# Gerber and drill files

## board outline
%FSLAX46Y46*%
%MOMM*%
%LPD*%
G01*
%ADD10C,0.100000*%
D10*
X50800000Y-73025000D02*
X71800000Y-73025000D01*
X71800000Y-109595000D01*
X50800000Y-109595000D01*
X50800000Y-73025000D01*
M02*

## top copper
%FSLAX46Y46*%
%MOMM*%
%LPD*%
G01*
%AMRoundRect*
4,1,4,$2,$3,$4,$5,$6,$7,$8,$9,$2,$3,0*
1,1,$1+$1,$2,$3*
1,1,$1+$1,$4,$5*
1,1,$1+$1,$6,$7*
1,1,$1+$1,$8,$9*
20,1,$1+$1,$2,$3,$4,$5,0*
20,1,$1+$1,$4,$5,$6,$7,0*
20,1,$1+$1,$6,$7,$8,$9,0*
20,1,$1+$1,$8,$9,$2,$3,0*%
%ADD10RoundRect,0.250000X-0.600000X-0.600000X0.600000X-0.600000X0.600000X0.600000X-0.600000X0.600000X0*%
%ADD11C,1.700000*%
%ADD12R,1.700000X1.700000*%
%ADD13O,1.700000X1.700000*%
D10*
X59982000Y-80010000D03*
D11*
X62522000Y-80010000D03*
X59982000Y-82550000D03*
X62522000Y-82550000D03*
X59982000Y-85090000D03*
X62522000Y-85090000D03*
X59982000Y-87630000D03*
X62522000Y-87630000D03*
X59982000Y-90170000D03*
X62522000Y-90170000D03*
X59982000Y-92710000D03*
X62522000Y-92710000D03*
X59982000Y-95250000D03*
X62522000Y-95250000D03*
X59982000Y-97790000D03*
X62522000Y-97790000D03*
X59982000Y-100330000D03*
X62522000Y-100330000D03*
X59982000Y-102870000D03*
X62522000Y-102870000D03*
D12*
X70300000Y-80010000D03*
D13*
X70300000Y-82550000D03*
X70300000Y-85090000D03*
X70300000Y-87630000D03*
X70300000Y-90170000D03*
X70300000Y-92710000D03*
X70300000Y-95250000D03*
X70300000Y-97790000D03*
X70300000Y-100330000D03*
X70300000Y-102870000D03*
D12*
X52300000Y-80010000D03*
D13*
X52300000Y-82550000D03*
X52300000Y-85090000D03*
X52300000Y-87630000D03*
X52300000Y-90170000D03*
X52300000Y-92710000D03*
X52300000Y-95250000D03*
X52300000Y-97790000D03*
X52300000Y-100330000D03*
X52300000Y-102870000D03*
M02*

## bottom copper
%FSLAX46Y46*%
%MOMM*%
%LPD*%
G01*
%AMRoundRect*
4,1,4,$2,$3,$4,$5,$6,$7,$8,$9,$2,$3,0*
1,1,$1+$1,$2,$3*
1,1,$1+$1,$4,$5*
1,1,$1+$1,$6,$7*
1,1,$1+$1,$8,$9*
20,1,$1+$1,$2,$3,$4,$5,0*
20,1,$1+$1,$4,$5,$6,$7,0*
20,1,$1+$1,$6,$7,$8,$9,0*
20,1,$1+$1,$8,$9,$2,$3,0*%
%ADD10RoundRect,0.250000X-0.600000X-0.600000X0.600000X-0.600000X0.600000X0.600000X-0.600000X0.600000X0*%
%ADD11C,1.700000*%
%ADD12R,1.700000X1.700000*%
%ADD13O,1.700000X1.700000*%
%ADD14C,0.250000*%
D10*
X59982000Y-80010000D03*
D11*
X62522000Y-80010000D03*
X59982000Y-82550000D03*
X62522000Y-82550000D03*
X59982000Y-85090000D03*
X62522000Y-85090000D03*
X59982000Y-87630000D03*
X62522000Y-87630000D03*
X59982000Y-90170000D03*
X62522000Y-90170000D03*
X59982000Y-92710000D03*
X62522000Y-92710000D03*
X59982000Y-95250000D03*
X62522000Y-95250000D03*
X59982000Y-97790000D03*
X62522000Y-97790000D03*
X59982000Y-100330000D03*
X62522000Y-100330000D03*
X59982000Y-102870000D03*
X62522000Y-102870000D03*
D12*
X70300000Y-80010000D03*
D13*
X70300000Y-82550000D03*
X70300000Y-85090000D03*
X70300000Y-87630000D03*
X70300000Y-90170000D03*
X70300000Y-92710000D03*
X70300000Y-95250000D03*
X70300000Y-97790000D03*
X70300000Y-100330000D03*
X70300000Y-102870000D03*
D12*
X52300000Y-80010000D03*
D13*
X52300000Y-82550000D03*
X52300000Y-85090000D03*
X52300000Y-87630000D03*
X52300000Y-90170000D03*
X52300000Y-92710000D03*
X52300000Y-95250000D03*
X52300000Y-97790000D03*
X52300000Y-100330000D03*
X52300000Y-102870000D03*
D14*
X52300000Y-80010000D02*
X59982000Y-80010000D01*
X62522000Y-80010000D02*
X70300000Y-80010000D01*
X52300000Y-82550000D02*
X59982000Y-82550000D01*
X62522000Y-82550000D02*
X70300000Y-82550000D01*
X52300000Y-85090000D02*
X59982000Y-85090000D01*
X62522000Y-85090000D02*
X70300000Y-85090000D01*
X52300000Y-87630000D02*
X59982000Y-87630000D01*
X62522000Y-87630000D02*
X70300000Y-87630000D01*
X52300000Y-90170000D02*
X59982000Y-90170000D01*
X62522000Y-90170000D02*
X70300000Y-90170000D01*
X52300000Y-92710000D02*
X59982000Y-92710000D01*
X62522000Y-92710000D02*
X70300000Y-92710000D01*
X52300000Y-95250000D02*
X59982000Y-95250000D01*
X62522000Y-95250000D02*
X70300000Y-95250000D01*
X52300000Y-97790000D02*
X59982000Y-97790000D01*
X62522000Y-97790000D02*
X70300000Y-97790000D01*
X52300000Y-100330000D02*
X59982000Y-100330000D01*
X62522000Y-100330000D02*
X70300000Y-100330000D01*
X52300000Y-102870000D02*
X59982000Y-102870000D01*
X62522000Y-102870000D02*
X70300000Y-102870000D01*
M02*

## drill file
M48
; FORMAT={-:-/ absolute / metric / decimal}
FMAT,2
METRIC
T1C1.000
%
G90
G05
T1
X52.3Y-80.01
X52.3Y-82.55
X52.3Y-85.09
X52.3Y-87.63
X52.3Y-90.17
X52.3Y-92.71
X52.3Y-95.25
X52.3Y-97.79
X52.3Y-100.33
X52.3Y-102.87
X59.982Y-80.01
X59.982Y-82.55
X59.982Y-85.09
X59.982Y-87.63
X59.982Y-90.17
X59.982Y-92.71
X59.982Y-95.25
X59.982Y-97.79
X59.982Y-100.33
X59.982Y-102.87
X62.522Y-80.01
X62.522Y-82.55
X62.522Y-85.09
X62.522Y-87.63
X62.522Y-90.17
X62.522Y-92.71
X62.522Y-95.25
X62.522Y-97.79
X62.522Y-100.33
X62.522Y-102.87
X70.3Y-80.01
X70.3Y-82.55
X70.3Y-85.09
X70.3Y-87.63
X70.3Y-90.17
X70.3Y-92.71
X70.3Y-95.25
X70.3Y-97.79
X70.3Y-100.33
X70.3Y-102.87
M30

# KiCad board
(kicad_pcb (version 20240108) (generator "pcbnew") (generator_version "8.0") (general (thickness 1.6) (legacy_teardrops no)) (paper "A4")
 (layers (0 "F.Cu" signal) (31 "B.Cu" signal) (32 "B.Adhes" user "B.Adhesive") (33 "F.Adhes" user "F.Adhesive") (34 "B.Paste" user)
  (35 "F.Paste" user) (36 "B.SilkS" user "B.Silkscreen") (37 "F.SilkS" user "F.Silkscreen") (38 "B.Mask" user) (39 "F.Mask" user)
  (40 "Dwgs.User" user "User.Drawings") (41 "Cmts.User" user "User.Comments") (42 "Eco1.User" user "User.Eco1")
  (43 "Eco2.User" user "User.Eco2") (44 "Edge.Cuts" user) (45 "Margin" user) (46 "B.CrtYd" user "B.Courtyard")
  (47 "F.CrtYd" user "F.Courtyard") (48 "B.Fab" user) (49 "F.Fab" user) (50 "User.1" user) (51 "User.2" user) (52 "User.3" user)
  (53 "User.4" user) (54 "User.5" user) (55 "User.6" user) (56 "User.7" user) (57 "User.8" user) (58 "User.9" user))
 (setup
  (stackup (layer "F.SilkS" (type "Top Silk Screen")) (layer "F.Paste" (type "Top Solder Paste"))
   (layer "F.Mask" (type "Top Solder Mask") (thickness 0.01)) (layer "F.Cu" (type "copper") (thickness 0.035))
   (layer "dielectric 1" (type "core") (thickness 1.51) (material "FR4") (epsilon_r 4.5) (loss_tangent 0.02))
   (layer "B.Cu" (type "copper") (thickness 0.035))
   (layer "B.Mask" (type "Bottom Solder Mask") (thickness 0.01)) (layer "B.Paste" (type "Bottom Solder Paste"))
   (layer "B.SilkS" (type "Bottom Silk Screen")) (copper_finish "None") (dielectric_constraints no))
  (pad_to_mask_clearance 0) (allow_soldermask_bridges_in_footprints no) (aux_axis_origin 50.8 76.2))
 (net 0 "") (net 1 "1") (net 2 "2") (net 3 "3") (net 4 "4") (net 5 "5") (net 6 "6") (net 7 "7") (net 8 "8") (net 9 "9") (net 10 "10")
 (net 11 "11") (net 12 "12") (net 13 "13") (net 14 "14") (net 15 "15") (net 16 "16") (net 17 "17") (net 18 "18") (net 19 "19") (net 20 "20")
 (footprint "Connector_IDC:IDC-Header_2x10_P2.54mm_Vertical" (layer "F.Cu") (at 59.982 80.01)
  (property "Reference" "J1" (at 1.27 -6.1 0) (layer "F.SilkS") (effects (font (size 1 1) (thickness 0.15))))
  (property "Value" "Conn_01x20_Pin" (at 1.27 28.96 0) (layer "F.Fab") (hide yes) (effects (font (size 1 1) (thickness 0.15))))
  (pad "1" thru_hole roundrect (at 0 0) (size 1.7 1.7) (drill 1) (layers "*.Cu" "*.Mask") (remove_unused_layers no)
   (roundrect_rratio 0.147059) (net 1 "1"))
  (pad "2" thru_hole circle (at 2.54 0) (size 1.7 1.7) (drill 1) (layers "*.Cu" "*.Mask") (remove_unused_layers no) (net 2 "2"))
  (pad "3" thru_hole circle (at 0 2.54) (size 1.7 1.7) (drill 1) (layers "*.Cu" "*.Mask") (remove_unused_layers no) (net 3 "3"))
  (pad "4" thru_hole circle (at 2.54 2.54) (size 1.7 1.7) (drill 1) (layers "*.Cu" "*.Mask") (remove_unused_layers no) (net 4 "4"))
  (pad "5" thru_hole circle (at 0 5.08) (size 1.7 1.7) (drill 1) (layers "*.Cu" "*.Mask") (remove_unused_layers no) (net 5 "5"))
  (pad "6" thru_hole circle (at 2.54 5.08) (size 1.7 1.7) (drill 1) (layers "*.Cu" "*.Mask") (remove_unused_layers no) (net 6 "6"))
  (pad "7" thru_hole circle (at 0 7.62) (size 1.7 1.7) (drill 1) (layers "*.Cu" "*.Mask") (remove_unused_layers no) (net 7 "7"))
  (pad "8" thru_hole circle (at 2.54 7.62) (size 1.7 1.7) (drill 1) (layers "*.Cu" "*.Mask") (remove_unused_layers no) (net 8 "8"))
  (pad "9" thru_hole circle (at 0 10.16) (size 1.7 1.7) (drill 1) (layers "*.Cu" "*.Mask") (remove_unused_layers no) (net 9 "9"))
  (pad "10" thru_hole circle (at 2.54 10.16) (size 1.7 1.7) (drill 1) (layers "*.Cu" "*.Mask") (remove_unused_layers no) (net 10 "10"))
  (pad "11" thru_hole circle (at 0 12.7) (size 1.7 1.7) (drill 1) (layers "*.Cu" "*.Mask") (remove_unused_layers no) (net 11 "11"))
  (pad "12" thru_hole circle (at 2.54 12.7) (size 1.7 1.7) (drill 1) (layers "*.Cu" "*.Mask") (remove_unused_layers no) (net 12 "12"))
  (pad "13" thru_hole circle (at 0 15.24) (size 1.7 1.7) (drill 1) (layers "*.Cu" "*.Mask") (remove_unused_layers no) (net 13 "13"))
  (pad "14" thru_hole circle (at 2.54 15.24) (size 1.7 1.7) (drill 1) (layers "*.Cu" "*.Mask") (remove_unused_layers no) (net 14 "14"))
  (pad "15" thru_hole circle (at 0 17.78) (size 1.7 1.7) (drill 1) (layers "*.Cu" "*.Mask") (remove_unused_layers no) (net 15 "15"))
  (pad "16" thru_hole circle (at 2.54 17.78) (size 1.7 1.7) (drill 1) (layers "*.Cu" "*.Mask") (remove_unused_layers no) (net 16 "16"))
  (pad "17" thru_hole circle (at 0 20.32) (size 1.7 1.7) (drill 1) (layers "*.Cu" "*.Mask") (remove_unused_layers no) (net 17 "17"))
  (pad "18" thru_hole circle (at 2.54 20.32) (size 1.7 1.7) (drill 1) (layers "*.Cu" "*.Mask") (remove_unused_layers no) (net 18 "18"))
  (pad "19" thru_hole circle (at 0 22.86) (size 1.7 1.7) (drill 1) (layers "*.Cu" "*.Mask") (remove_unused_layers no) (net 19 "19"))
  (pad "20" thru_hole circle (at 2.54 22.86) (size 1.7 1.7) (drill 1) (layers "*.Cu" "*.Mask") (remove_unused_layers no) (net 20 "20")))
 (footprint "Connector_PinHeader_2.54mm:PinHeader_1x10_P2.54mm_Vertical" (layer "B.Cu") (at 70.3 80.01 180)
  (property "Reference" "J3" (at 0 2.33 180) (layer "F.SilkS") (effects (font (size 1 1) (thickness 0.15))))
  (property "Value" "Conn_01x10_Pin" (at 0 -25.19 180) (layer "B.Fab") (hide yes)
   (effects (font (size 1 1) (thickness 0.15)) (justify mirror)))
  (pad "1" thru_hole rect (at 0 0 180) (size 1.7 1.7) (drill 1) (layers "*.Cu" "*.Mask") (remove_unused_layers no) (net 2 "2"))
  (pad "2" thru_hole oval (at 0 -2.54 180) (size 1.7 1.7) (drill 1) (layers "*.Cu" "*.Mask") (remove_unused_layers no) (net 4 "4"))
  (pad "3" thru_hole oval (at 0 -5.08 180) (size 1.7 1.7) (drill 1) (layers "*.Cu" "*.Mask") (remove_unused_layers no) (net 6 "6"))
  (pad "4" thru_hole oval (at 0 -7.62 180) (size 1.7 1.7) (drill 1) (layers "*.Cu" "*.Mask") (remove_unused_layers no) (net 8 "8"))
  (pad "5" thru_hole oval (at 0 -10.16 180) (size 1.7 1.7) (drill 1) (layers "*.Cu" "*.Mask") (remove_unused_layers no) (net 10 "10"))
  (pad "6" thru_hole oval (at 0 -12.7 180) (size 1.7 1.7) (drill 1) (layers "*.Cu" "*.Mask") (remove_unused_layers no) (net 12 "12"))
  (pad "7" thru_hole oval (at 0 -15.24 180) (size 1.7 1.7) (drill 1) (layers "*.Cu" "*.Mask") (remove_unused_layers no) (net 14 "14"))
  (pad "8" thru_hole oval (at 0 -17.78 180) (size 1.7 1.7) (drill 1) (layers "*.Cu" "*.Mask") (remove_unused_layers no) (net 16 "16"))
  (pad "9" thru_hole oval (at 0 -20.32 180) (size 1.7 1.7) (drill 1) (layers "*.Cu" "*.Mask") (remove_unused_layers no) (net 18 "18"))
  (pad "10" thru_hole oval (at 0 -22.86 180) (size 1.7 1.7) (drill 1) (layers "*.Cu" "*.Mask") (remove_unused_layers no) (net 20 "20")))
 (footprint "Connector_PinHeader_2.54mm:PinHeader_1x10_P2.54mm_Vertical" (layer "B.Cu") (at 52.3 80.01 180)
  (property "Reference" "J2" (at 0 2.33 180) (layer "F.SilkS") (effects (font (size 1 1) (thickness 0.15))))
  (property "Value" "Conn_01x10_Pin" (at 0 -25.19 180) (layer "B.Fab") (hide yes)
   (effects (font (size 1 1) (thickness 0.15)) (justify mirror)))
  (pad "1" thru_hole rect (at 0 0 180) (size 1.7 1.7) (drill 1) (layers "*.Cu" "*.Mask") (remove_unused_layers no) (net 1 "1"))
  (pad "2" thru_hole oval (at 0 -2.54 180) (size 1.7 1.7) (drill 1) (layers "*.Cu" "*.Mask") (remove_unused_layers no) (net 3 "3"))
  (pad "3" thru_hole oval (at 0 -5.08 180) (size 1.7 1.7) (drill 1) (layers "*.Cu" "*.Mask") (remove_unused_layers no) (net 5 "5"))
  (pad "4" thru_hole oval (at 0 -7.62 180) (size 1.7 1.7) (drill 1) (layers "*.Cu" "*.Mask") (remove_unused_layers no) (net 7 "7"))
  (pad "5" thru_hole oval (at 0 -10.16 180) (size 1.7 1.7) (drill 1) (layers "*.Cu" "*.Mask") (remove_unused_layers no) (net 9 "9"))
  (pad "6" thru_hole oval (at 0 -12.7 180) (size 1.7 1.7) (drill 1) (layers "*.Cu" "*.Mask") (remove_unused_layers no) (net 11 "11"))
  (pad "7" thru_hole oval (at 0 -15.24 180) (size 1.7 1.7) (drill 1) (layers "*.Cu" "*.Mask") (remove_unused_layers no) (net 13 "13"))
  (pad "8" thru_hole oval (at 0 -17.78 180) (size 1.7 1.7) (drill 1) (layers "*.Cu" "*.Mask") (remove_unused_layers no) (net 15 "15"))
  (pad "9" thru_hole oval (at 0 -20.32 180) (size 1.7 1.7) (drill 1) (layers "*.Cu" "*.Mask") (remove_unused_layers no) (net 17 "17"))
  (pad "10" thru_hole oval (at 0 -22.86 180) (size 1.7 1.7) (drill 1) (layers "*.Cu" "*.Mask") (remove_unused_layers no) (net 19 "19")))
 (gr_rect (start 50.8 73.025) (end 71.8 109.595) (stroke (width 0.1) (type default)) (fill none) (layer "Edge.Cuts"))
 (segment (start 52.3 80.01) (end 59.982 80.01) (width 0.25) (layer "B.Cu") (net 1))
 (segment (start 62.522 80.01) (end 70.3 80.01) (width 0.25) (layer "B.Cu") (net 2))
 (segment (start 52.3 82.55) (end 59.982 82.55) (width 0.25) (layer "B.Cu") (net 3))
 (segment (start 62.522 82.55) (end 70.3 82.55) (width 0.25) (layer "B.Cu") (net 4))
 (segment (start 52.3 85.09) (end 59.982 85.09) (width 0.25) (layer "B.Cu") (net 5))
 (segment (start 62.522 85.09) (end 70.3 85.09) (width 0.25) (layer "B.Cu") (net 6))
 (segment (start 52.3 87.63) (end 59.982 87.63) (width 0.25) (layer "B.Cu") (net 7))
 (segment (start 62.522 87.63) (end 70.3 87.63) (width 0.25) (layer "B.Cu") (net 8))
 (segment (start 52.3 90.17) (end 59.982 90.17) (width 0.25) (layer "B.Cu") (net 9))
 (segment (start 62.522 90.17) (end 70.3 90.17) (width 0.25) (layer "B.Cu") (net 10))
 (segment (start 52.3 92.71) (end 59.982 92.71) (width 0.25) (layer "B.Cu") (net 11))
 (segment (start 62.522 92.71) (end 70.3 92.71) (width 0.25) (layer "B.Cu") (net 12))
 (segment (start 52.3 95.25) (end 59.982 95.25) (width 0.25) (layer "B.Cu") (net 13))
 (segment (start 62.522 95.25) (end 70.3 95.25) (width 0.25) (layer "B.Cu") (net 14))
 (segment (start 52.3 97.79) (end 59.982 97.79) (width 0.25) (layer "B.Cu") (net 15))
 (segment (start 62.522 97.79) (end 70.3 97.79) (width 0.25) (layer "B.Cu") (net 16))
 (segment (start 52.3 100.33) (end 59.982 100.33) (width 0.25) (layer "B.Cu") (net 17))
 (segment (start 62.522 100.33) (end 70.3 100.33) (width 0.25) (layer "B.Cu") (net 18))
 (segment (start 52.3 102.87) (end 59.982 102.87) (width 0.25) (layer "B.Cu") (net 19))
 (segment (start 62.522 102.87) (end 70.3 102.87) (width 0.25) (layer "B.Cu") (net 20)))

